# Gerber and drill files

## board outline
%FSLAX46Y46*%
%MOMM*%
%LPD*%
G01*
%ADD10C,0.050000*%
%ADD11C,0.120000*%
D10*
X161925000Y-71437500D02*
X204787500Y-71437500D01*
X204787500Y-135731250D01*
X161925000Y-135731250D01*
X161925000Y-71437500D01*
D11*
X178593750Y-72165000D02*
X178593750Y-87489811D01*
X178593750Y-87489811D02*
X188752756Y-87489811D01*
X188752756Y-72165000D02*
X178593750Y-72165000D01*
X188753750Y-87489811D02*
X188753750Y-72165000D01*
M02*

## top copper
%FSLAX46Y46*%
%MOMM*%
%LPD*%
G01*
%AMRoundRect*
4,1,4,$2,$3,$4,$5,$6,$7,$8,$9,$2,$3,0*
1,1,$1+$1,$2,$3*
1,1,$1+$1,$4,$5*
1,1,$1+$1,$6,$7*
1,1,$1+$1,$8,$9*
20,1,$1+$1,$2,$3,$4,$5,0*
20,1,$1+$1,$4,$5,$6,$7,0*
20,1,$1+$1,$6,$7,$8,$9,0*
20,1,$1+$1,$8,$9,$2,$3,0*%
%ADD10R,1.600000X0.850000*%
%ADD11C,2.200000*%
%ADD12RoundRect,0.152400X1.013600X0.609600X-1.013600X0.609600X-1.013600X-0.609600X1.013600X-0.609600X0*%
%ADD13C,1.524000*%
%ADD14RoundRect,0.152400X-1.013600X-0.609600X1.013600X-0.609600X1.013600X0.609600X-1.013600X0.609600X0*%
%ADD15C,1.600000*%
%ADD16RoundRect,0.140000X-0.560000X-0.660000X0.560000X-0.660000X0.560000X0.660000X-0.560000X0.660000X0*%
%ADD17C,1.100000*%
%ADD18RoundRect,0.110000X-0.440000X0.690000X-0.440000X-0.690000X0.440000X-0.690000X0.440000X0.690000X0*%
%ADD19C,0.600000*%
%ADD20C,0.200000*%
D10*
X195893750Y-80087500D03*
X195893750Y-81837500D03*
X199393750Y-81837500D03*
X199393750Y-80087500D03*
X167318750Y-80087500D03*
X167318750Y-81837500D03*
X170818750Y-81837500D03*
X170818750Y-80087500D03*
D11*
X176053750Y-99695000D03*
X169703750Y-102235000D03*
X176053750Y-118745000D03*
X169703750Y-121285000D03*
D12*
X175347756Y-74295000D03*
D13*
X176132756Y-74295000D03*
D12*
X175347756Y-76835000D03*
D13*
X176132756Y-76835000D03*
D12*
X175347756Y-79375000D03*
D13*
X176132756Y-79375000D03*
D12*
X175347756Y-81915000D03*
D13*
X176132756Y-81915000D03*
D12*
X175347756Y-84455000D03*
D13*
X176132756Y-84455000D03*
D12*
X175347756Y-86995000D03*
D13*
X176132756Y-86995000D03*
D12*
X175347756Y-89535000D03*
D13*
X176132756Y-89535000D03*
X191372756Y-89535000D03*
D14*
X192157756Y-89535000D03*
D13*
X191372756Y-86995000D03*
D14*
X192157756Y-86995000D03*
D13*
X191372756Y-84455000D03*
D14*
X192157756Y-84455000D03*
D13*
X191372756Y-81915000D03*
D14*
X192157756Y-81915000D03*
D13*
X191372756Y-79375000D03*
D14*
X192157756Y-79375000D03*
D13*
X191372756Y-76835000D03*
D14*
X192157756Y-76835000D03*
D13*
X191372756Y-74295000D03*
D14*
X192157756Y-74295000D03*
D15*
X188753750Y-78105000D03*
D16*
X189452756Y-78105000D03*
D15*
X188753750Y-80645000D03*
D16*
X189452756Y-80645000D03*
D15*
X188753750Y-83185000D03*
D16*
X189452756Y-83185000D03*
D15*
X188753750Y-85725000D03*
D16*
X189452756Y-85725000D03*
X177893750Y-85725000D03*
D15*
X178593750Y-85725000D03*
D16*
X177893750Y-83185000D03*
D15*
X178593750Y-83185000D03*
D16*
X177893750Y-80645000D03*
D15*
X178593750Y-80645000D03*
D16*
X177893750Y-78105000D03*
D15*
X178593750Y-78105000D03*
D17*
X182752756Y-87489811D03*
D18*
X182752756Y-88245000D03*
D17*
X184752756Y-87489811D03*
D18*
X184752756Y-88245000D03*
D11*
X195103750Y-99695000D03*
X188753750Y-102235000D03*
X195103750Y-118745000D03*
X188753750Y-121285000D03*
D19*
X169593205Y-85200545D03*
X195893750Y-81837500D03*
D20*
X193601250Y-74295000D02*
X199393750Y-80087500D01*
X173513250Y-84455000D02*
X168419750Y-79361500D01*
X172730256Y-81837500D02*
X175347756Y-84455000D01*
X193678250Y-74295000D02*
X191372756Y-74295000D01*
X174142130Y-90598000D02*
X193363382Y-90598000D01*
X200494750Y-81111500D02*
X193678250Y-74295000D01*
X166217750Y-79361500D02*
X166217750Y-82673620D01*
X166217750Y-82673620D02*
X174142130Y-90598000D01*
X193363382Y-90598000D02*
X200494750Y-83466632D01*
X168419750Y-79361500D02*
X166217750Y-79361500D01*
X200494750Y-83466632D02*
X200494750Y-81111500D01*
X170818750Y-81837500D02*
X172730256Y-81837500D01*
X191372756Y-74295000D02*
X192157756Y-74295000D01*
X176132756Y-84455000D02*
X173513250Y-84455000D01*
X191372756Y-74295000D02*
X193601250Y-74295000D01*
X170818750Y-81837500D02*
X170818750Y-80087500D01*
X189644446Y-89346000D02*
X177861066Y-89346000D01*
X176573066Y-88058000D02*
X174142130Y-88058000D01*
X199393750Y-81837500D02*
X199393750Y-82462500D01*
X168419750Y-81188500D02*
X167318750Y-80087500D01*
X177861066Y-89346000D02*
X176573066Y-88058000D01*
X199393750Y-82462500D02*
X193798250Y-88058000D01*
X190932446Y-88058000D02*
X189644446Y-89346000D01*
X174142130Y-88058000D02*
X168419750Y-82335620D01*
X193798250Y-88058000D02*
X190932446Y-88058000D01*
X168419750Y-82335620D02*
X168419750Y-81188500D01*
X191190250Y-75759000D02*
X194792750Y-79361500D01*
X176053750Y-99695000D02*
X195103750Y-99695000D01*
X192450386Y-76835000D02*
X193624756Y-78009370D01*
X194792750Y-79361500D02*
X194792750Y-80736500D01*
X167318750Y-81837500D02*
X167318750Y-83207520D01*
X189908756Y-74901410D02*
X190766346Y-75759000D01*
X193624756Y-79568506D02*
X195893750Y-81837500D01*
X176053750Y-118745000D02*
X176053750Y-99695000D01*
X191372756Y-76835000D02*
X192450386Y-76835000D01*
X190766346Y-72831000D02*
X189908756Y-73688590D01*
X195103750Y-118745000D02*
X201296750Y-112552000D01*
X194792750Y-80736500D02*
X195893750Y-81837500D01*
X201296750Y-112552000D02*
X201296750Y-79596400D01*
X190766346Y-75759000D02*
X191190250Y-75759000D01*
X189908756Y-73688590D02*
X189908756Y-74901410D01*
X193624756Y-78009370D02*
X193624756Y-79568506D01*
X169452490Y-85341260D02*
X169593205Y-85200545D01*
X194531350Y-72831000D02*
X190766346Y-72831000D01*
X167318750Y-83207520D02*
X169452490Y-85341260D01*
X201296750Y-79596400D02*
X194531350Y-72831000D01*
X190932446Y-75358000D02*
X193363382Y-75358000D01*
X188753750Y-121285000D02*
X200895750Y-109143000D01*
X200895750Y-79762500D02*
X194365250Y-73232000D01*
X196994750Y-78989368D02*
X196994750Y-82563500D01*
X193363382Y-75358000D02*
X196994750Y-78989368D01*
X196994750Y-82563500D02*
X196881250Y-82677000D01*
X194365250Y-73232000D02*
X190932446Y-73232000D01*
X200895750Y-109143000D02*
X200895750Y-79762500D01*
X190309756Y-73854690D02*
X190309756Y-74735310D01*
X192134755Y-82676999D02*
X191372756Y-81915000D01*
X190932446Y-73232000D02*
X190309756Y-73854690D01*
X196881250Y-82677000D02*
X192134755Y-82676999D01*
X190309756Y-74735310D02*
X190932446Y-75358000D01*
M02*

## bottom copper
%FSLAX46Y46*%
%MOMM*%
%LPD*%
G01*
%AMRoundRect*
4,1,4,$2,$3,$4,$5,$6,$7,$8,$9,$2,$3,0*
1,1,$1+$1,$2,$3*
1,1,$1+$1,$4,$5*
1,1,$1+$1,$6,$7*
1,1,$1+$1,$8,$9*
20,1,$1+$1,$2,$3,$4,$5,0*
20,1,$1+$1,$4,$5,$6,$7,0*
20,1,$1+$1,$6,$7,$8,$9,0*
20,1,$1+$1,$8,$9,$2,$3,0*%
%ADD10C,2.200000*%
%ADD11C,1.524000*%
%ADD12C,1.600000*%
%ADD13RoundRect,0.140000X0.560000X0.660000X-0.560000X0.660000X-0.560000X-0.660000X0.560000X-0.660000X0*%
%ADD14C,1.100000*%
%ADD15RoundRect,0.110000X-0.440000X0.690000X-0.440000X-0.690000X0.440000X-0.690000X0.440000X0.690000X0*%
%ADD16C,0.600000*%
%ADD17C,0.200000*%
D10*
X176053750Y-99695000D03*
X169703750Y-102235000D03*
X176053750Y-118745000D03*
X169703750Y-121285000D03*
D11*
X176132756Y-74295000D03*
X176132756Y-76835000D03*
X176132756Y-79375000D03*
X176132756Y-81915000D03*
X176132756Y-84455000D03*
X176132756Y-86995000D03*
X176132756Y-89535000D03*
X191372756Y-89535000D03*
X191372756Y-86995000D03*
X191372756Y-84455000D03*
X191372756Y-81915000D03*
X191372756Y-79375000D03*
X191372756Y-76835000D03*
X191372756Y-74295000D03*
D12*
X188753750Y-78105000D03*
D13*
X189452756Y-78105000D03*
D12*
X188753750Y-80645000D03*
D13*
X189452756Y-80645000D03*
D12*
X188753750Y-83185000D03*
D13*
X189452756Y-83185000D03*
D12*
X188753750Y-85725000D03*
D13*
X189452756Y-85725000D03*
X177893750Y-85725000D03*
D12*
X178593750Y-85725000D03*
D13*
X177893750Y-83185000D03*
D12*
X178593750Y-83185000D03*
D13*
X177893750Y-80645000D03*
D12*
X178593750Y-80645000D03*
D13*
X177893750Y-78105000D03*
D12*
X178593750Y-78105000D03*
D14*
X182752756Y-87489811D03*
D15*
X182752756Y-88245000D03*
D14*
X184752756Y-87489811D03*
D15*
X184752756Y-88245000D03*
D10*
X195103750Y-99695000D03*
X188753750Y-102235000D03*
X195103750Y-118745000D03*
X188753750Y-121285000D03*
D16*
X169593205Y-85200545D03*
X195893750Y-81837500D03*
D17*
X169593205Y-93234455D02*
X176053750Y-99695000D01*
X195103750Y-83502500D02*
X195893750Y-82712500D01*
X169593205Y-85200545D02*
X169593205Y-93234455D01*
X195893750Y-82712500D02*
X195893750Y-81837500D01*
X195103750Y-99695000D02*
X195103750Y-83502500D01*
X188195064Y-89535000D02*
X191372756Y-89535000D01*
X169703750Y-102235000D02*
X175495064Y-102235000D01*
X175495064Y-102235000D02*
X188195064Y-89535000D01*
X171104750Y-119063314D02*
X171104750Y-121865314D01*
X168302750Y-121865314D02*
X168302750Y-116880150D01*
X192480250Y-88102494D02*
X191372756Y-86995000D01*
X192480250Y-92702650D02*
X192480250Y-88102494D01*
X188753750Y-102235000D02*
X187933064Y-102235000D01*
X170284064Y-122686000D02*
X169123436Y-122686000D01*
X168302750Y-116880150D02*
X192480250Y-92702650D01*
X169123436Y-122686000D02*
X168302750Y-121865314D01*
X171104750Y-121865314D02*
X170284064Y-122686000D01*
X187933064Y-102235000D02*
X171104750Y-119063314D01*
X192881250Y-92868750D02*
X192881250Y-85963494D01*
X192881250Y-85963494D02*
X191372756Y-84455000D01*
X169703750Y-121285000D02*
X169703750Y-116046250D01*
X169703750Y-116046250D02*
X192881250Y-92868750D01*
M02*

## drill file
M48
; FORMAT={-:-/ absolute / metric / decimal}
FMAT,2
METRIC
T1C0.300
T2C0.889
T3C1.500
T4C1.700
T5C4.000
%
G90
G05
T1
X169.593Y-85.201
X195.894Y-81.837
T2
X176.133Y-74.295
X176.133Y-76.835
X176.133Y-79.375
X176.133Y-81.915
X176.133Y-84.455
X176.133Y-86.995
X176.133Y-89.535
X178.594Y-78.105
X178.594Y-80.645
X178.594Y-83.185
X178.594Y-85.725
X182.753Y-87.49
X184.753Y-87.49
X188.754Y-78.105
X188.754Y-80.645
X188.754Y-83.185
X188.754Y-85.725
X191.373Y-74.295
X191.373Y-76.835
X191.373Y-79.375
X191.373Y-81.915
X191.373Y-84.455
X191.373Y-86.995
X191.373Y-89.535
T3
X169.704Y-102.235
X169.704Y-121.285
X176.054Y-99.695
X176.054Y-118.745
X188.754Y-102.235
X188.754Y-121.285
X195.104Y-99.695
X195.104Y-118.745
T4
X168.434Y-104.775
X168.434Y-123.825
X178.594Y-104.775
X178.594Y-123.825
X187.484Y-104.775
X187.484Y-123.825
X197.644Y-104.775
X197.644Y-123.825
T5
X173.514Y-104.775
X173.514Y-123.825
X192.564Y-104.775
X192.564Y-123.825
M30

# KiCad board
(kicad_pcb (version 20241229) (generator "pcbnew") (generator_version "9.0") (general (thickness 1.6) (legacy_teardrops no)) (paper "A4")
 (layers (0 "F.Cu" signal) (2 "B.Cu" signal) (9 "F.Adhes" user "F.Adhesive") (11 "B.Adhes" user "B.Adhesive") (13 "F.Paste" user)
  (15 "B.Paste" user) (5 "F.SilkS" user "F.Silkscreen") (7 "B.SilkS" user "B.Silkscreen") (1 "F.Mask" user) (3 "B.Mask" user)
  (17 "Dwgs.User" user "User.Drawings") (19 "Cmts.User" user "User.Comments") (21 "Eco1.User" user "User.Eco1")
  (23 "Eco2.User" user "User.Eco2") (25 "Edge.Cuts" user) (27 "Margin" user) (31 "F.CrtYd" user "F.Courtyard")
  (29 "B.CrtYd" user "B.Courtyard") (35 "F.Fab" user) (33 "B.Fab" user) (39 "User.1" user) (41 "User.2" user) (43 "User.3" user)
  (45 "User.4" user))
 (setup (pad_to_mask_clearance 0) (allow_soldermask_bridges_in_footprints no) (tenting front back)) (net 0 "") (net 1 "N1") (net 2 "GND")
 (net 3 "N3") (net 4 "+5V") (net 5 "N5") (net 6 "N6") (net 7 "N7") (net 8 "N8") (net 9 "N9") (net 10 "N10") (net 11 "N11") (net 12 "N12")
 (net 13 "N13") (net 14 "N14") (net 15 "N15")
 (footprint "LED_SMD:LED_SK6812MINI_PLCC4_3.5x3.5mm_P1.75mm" (layer "F.Cu") (at 197.64375 80.9625)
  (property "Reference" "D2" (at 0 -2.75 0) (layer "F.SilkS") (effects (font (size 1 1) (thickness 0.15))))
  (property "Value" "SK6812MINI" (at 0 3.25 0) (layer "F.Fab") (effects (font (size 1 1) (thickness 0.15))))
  (pad "1" smd rect (at -1.75 -0.875) (size 1.6 0.85) (layers "F.Cu" "F.Mask" "F.Paste") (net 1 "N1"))
  (pad "2" smd rect (at -1.75 0.875) (size 1.6 0.85) (layers "F.Cu" "F.Mask" "F.Paste") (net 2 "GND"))
  (pad "3" smd rect (at 1.75 0.875) (size 1.6 0.85) (layers "F.Cu" "F.Mask" "F.Paste") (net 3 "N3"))
  (pad "4" smd rect (at 1.75 -0.875) (size 1.6 0.85) (layers "F.Cu" "F.Mask" "F.Paste") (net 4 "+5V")))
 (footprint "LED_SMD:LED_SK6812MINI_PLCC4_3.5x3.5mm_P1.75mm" (layer "F.Cu") (at 169.06875 80.9625)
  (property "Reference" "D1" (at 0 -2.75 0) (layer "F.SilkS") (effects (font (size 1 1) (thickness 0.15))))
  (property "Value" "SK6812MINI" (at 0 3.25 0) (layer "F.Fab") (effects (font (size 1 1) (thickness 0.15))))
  (pad "1" smd rect (at -1.75 -0.875) (size 1.6 0.85) (layers "F.Cu" "F.Mask" "F.Paste") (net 3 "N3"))
  (pad "2" smd rect (at -1.75 0.875) (size 1.6 0.85) (layers "F.Cu" "F.Mask" "F.Paste") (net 2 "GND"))
  (pad "3" smd rect (at 1.75 0.875) (size 1.6 0.85) (layers "F.Cu" "F.Mask" "F.Paste") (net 4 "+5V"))
  (pad "4" smd rect (at 1.75 -0.875) (size 1.6 0.85) (layers "F.Cu" "F.Mask" "F.Paste") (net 4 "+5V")))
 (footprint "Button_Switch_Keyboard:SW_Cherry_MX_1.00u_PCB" (layer "F.Cu") (at 176.05375 99.695)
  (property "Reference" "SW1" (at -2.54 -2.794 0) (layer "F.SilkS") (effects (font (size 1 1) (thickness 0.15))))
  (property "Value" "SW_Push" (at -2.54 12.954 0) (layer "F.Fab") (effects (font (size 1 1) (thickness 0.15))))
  (pad "" np_thru_hole circle (at -7.62 5.08) (size 1.7 1.7) (drill 1.7) (layers "*.Cu" "*.Mask"))
  (pad "" np_thru_hole circle (at -2.54 5.08) (size 4 4) (drill 4) (layers "*.Cu" "*.Mask"))
  (pad "" np_thru_hole circle (at 2.54 5.08) (size 1.7 1.7) (drill 1.7) (layers "*.Cu" "*.Mask"))
  (pad "1" thru_hole circle (at 0 0) (size 2.2 2.2) (drill 1.5) (layers "*.Cu" "*.Mask") (remove_unused_layers no) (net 2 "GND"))
  (pad "2" thru_hole circle (at -6.35 2.54) (size 2.2 2.2) (drill 1.5) (layers "*.Cu" "*.Mask") (remove_unused_layers no) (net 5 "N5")))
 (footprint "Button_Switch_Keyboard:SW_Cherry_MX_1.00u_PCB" (layer "F.Cu") (at 176.05375 118.745)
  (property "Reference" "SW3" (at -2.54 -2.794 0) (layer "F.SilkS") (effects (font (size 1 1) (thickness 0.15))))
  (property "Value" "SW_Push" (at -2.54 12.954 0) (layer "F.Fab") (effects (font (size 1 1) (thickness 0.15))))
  (pad "" np_thru_hole circle (at -7.62 5.08) (size 1.7 1.7) (drill 1.7) (layers "*.Cu" "*.Mask"))
  (pad "" np_thru_hole circle (at -2.54 5.08) (size 4 4) (drill 4) (layers "*.Cu" "*.Mask"))
  (pad "" np_thru_hole circle (at 2.54 5.08) (size 1.7 1.7) (drill 1.7) (layers "*.Cu" "*.Mask"))
  (pad "1" thru_hole circle (at 0 0) (size 2.2 2.2) (drill 1.5) (layers "*.Cu" "*.Mask") (remove_unused_layers no) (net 2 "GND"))
  (pad "2" thru_hole circle (at -6.35 2.54) (size 2.2 2.2) (drill 1.5) (layers "*.Cu" "*.Mask") (remove_unused_layers no) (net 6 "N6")))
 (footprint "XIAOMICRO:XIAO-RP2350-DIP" (layer "F.Cu") (at 183.75375 81.8515)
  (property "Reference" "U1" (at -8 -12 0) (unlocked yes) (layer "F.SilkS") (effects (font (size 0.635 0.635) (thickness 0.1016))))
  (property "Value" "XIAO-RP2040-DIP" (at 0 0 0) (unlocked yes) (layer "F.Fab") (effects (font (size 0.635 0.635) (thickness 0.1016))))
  (fp_line (start -5.16 -9.6865) (end -5.16 5.638311) (stroke (width 0.12) (type default)) (layer "Edge.Cuts"))
  (fp_line (start -5.16 5.638311) (end 4.999006 5.638311) (stroke (width 0.12) (type default)) (layer "Edge.Cuts"))
  (fp_line (start 4.999006 -9.6865) (end -5.16 -9.6865) (stroke (width 0.12) (type default)) (layer "Edge.Cuts"))
  (fp_line (start 5 5.638311) (end 5 -9.6865) (stroke (width 0.12) (type default)) (layer "Edge.Cuts"))
  (pad "1" smd roundrect (at -8.405994 -7.5565 180) (size 2.332 1.524) (layers "F.Cu" "F.Mask") (roundrect_rratio 0.1) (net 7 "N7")
   (thermal_bridge_angle 45))
  (pad "1" thru_hole circle (at -7.620994 -7.5565 180) (size 1.524 1.524) (drill 0.889) (layers "*.Cu" "*.Mask") (remove_unused_layers no)
   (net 7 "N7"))
  (pad "2" smd roundrect (at -8.405994 -5.0165 180) (size 2.332 1.524) (layers "F.Cu" "F.Mask") (roundrect_rratio 0.1) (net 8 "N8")
   (thermal_bridge_angle 45))
  (pad "2" thru_hole circle (at -7.620994 -5.0165 180) (size 1.524 1.524) (drill 0.889) (layers "*.Cu" "*.Mask") (remove_unused_layers no)
   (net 8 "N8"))
  (pad "3" smd roundrect (at -8.405994 -2.4765 180) (size 2.332 1.524) (layers "F.Cu" "F.Mask") (roundrect_rratio 0.1) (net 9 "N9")
   (thermal_bridge_angle 45))
  (pad "3" thru_hole circle (at -7.620994 -2.4765 180) (size 1.524 1.524) (drill 0.889) (layers "*.Cu" "*.Mask") (remove_unused_layers no)
   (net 9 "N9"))
  (pad "4" smd roundrect (at -8.405994 0.0635 180) (size 2.332 1.524) (layers "F.Cu" "F.Mask") (roundrect_rratio 0.1) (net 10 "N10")
   (thermal_bridge_angle 45))
  (pad "4" thru_hole circle (at -7.620994 0.0635 180) (size 1.524 1.524) (drill 0.889) (layers "*.Cu" "*.Mask") (remove_unused_layers no)
   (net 10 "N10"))
  (pad "5" smd roundrect (at -8.405994 2.6035 180) (size 2.332 1.524) (layers "F.Cu" "F.Mask") (roundrect_rratio 0.1) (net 4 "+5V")
   (thermal_bridge_angle 45))
  (pad "5" thru_hole circle (at -7.620994 2.6035 180) (size 1.524 1.524) (drill 0.889) (layers "*.Cu" "*.Mask") (remove_unused_layers no)
   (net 4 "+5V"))
  (pad "6" smd roundrect (at -8.405994 5.1435 180) (size 2.332 1.524) (layers "F.Cu" "F.Mask") (roundrect_rratio 0.1) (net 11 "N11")
   (thermal_bridge_angle 45))
  (pad "6" thru_hole circle (at -7.620994 5.1435 180) (size 1.524 1.524) (drill 0.889) (layers "*.Cu" "*.Mask") (remove_unused_layers no)
   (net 11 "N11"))
  (pad "7" smd roundrect (at -8.405994 7.6835 180) (size 2.332 1.524) (layers "F.Cu" "F.Mask") (roundrect_rratio 0.1) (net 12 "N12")
   (thermal_bridge_angle 45))
  (pad "7" thru_hole circle (at -7.620994 7.6835 180) (size 1.524 1.524) (drill 0.889) (layers "*.Cu" "*.Mask") (remove_unused_layers no)
   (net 12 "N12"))
  (pad "8" thru_hole circle (at 7.619006 7.6835) (size 1.524 1.524) (drill 0.889) (layers "*.Cu" "*.Mask") (remove_unused_layers no)
   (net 5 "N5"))
  (pad "8" smd roundrect (at 8.404006 7.6835) (size 2.332 1.524) (layers "F.Cu" "F.Mask") (roundrect_rratio 0.1) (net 5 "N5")
   (thermal_bridge_angle 45))
  (pad "9" thru_hole circle (at 7.619006 5.1435) (size 1.524 1.524) (drill 0.889) (layers "*.Cu" "*.Mask") (remove_unused_layers no)
   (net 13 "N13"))
  (pad "9" smd roundrect (at 8.404006 5.1435) (size 2.332 1.524) (layers "F.Cu" "F.Mask") (roundrect_rratio 0.1) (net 13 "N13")
   (thermal_bridge_angle 45))
  (pad "10" thru_hole circle (at 7.619006 2.6035) (size 1.524 1.524) (drill 0.889) (layers "*.Cu" "*.Mask") (remove_unused_layers no)
   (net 6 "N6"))
  (pad "10" smd roundrect (at 8.404006 2.6035) (size 2.332 1.524) (layers "F.Cu" "F.Mask") (roundrect_rratio 0.1) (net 6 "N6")
   (thermal_bridge_angle 45))
  (pad "11" thru_hole circle (at 7.619006 0.0635) (size 1.524 1.524) (drill 0.889) (layers "*.Cu" "*.Mask") (remove_unused_layers no)
   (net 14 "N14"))
  (pad "11" smd roundrect (at 8.404006 0.0635) (size 2.332 1.524) (layers "F.Cu" "F.Mask") (roundrect_rratio 0.1) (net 14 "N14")
   (thermal_bridge_angle 45))
  (pad "12" thru_hole circle (at 7.619006 -2.4765) (size 1.524 1.524) (drill 0.889) (layers "*.Cu" "*.Mask") (remove_unused_layers no)
   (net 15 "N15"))
  (pad "12" smd roundrect (at 8.404006 -2.4765) (size 2.332 1.524) (layers "F.Cu" "F.Mask") (roundrect_rratio 0.1) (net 15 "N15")
   (thermal_bridge_angle 45))
  (pad "13" thru_hole circle (at 7.619006 -5.0165) (size 1.524 1.524) (drill 0.889) (layers "*.Cu" "*.Mask") (remove_unused_layers no)
   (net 2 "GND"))
  (pad "13" smd roundrect (at 8.404006 -5.0165) (size 2.332 1.524) (layers "F.Cu" "F.Mask") (roundrect_rratio 0.1) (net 2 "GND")
   (thermal_bridge_angle 45))
  (pad "14" thru_hole circle (at 7.619006 -7.5565) (size 1.524 1.524) (drill 0.889) (layers "*.Cu" "*.Mask") (remove_unused_layers no)
   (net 4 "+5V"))
  (pad "14" smd roundrect (at 8.404006 -7.5565) (size 2.332 1.524) (layers "F.Cu" "F.Mask") (roundrect_rratio 0.1) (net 4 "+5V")
   (thermal_bridge_angle 45))
  (pad "15" thru_hole circle (at 5 -3.7465 180) (size 1.6 1.6) (drill 0.889) (layers "*.Cu" "*.Mask") (remove_unused_layers no))
  (pad "15" smd roundrect (at 5.699006 -3.7465) (size 1.4 1.6) (layers "F.Cu" "F.Mask") (roundrect_rratio 0.1) (thermal_bridge_angle 45))
  (pad "15" smd roundrect (at 5.699006 -3.7465 180) (size 1.4 1.6) (layers "B.Cu" "B.Mask" "B.Paste") (roundrect_rratio 0.1)
   (thermal_bridge_angle 45))
  (pad "16" thru_hole circle (at 5 -1.2065 180) (size 1.6 1.6) (drill 0.889) (layers "*.Cu" "*.Mask") (remove_unused_layers no))
  (pad "16" smd roundrect (at 5.699006 -1.2065) (size 1.4 1.6) (layers "F.Cu" "F.Mask") (roundrect_rratio 0.1) (thermal_bridge_angle 45))
  (pad "16" smd roundrect (at 5.699006 -1.2065 180) (size 1.4 1.6) (layers "B.Cu" "B.Mask" "B.Paste") (roundrect_rratio 0.1)
   (thermal_bridge_angle 45))
  (pad "17" thru_hole circle (at 5 1.3335 180) (size 1.6 1.6) (drill 0.889) (layers "*.Cu" "*.Mask") (remove_unused_layers no))
  (pad "17" smd roundrect (at 5.699006 1.3335) (size 1.4 1.6) (layers "F.Cu" "F.Mask") (roundrect_rratio 0.1) (thermal_bridge_angle 45))
  (pad "17" smd roundrect (at 5.699006 1.3335 180) (size 1.4 1.6) (layers "B.Cu" "B.Mask" "B.Paste") (roundrect_rratio 0.1)
   (thermal_bridge_angle 45))
  (pad "18" thru_hole circle (at 5 3.8735 180) (size 1.6 1.6) (drill 0.889) (layers "*.Cu" "*.Mask") (remove_unused_layers no))
  (pad "18" smd roundrect (at 5.699006 3.8735) (size 1.4 1.6) (layers "F.Cu" "F.Mask") (roundrect_rratio 0.1) (thermal_bridge_angle 45))
  (pad "18" smd roundrect (at 5.699006 3.8735 180) (size 1.4 1.6) (layers "B.Cu" "B.Mask" "B.Paste") (roundrect_rratio 0.1)
   (thermal_bridge_angle 45))
  (pad "19" smd roundrect (at -5.86 3.8735) (size 1.4 1.6) (layers "F.Cu" "F.Mask") (roundrect_rratio 0.1) (thermal_bridge_angle 45))
  (pad "19" smd roundrect (at -5.86 3.8735 180) (size 1.4 1.6) (layers "B.Cu" "B.Mask" "B.Paste") (roundrect_rratio 0.1)
   (thermal_bridge_angle 45))
  (pad "19" thru_hole circle (at -5.16 3.8735 180) (size 1.6 1.6) (drill 0.889) (layers "*.Cu" "*.Mask") (remove_unused_layers no))
  (pad "20" smd roundrect (at -5.86 1.3335) (size 1.4 1.6) (layers "F.Cu" "F.Mask") (roundrect_rratio 0.1) (thermal_bridge_angle 45))
  (pad "20" smd roundrect (at -5.86 1.3335 180) (size 1.4 1.6) (layers "B.Cu" "B.Mask" "B.Paste") (roundrect_rratio 0.1)
   (thermal_bridge_angle 45))
  (pad "20" thru_hole circle (at -5.16 1.3335 180) (size 1.6 1.6) (drill 0.889) (layers "*.Cu" "*.Mask") (remove_unused_layers no))
  (pad "21" smd roundrect (at -5.86 -1.2065) (size 1.4 1.6) (layers "F.Cu" "F.Mask") (roundrect_rratio 0.1) (thermal_bridge_angle 45))
  (pad "21" smd roundrect (at -5.86 -1.2065 180) (size 1.4 1.6) (layers "B.Cu" "B.Mask" "B.Paste") (roundrect_rratio 0.1)
   (thermal_bridge_angle 45))
  (pad "21" thru_hole circle (at -5.16 -1.2065 180) (size 1.6 1.6) (drill 0.889) (layers "*.Cu" "*.Mask") (remove_unused_layers no))
  (pad "22" smd roundrect (at -5.86 -3.7465) (size 1.4 1.6) (layers "F.Cu" "F.Mask") (roundrect_rratio 0.1) (thermal_bridge_angle 45))
  (pad "22" smd roundrect (at -5.86 -3.7465 180) (size 1.4 1.6) (layers "B.Cu" "B.Mask" "B.Paste") (roundrect_rratio 0.1)
   (thermal_bridge_angle 45))
  (pad "22" thru_hole circle (at -5.16 -3.7465 180) (size 1.6 1.6) (drill 0.889) (layers "*.Cu" "*.Mask") (remove_unused_layers no))
  (pad "23" thru_hole circle (at -1.000994 5.638311 180) (size 1.1 1.1) (drill 0.889) (layers "*.Cu" "*.Mask") (remove_unused_layers no))
  (pad "23" smd roundrect (at -1.000994 6.3935 270) (size 1.6 1.1) (layers "F.Cu" "F.Mask") (roundrect_rratio 0.1) (thermal_bridge_angle 45))
  (pad "23" smd roundrect (at -1.000994 6.3935 270) (size 1.6 1.1) (layers "B.Cu" "B.Mask" "B.Paste") (roundrect_rratio 0.1)
   (thermal_bridge_angle 45))
  (pad "24" thru_hole circle (at 0.999006 5.638311 180) (size 1.1 1.1) (drill 0.889) (layers "*.Cu" "*.Mask") (remove_unused_layers no))
  (pad "24" smd roundrect (at 0.999006 6.3935 270) (size 1.6 1.1) (layers "F.Cu" "F.Mask") (roundrect_rratio 0.1) (thermal_bridge_angle 45))
  (pad "24" smd roundrect (at 0.999006 6.3935 270) (size 1.6 1.1) (layers "B.Cu" "B.Mask" "B.Paste") (roundrect_rratio 0.1)
   (thermal_bridge_angle 45)))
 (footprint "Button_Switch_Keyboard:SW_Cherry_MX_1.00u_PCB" (layer "F.Cu") (at 195.10375 99.695)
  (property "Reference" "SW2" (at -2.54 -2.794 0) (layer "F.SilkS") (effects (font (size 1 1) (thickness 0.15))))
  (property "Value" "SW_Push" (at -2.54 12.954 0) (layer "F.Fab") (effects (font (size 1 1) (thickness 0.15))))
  (pad "" np_thru_hole circle (at -7.62 5.08) (size 1.7 1.7) (drill 1.7) (layers "*.Cu" "*.Mask"))
  (pad "" np_thru_hole circle (at -2.54 5.08) (size 4 4) (drill 4) (layers "*.Cu" "*.Mask"))
  (pad "" np_thru_hole circle (at 2.54 5.08) (size 1.7 1.7) (drill 1.7) (layers "*.Cu" "*.Mask"))
  (pad "1" thru_hole circle (at 0 0) (size 2.2 2.2) (drill 1.5) (layers "*.Cu" "*.Mask") (remove_unused_layers no) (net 2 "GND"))
  (pad "2" thru_hole circle (at -6.35 2.54) (size 2.2 2.2) (drill 1.5) (layers "*.Cu" "*.Mask") (remove_unused_layers no) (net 13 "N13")))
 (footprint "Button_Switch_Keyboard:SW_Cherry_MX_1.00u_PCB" (layer "F.Cu") (at 195.10375 118.745)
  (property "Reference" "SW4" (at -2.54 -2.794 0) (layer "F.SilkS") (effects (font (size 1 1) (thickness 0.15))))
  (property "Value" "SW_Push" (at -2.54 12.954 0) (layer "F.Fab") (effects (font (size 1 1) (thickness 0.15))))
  (pad "" np_thru_hole circle (at -7.62 5.08) (size 1.7 1.7) (drill 1.7) (layers "*.Cu" "*.Mask"))
  (pad "" np_thru_hole circle (at -2.54 5.08) (size 4 4) (drill 4) (layers "*.Cu" "*.Mask"))
  (pad "" np_thru_hole circle (at 2.54 5.08) (size 1.7 1.7) (drill 1.7) (layers "*.Cu" "*.Mask"))
  (pad "1" thru_hole circle (at 0 0) (size 2.2 2.2) (drill 1.5) (layers "*.Cu" "*.Mask") (remove_unused_layers no) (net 2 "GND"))
  (pad "2" thru_hole circle (at -6.35 2.54) (size 2.2 2.2) (drill 1.5) (layers "*.Cu" "*.Mask") (remove_unused_layers no) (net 14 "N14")))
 (gr_rect (start 161.925 71.4375) (end 204.7875 135.73125) (stroke (width 0.05) (type default)) (fill no) (layer "Edge.Cuts"))
 (segment (start 193.60125 74.295) (end 199.39375 80.0875) (width 0.2) (layer "F.Cu") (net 4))
 (segment (start 173.51325 84.455) (end 168.41975 79.3615) (width 0.2) (layer "F.Cu") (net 4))
 (segment (start 172.730256 81.8375) (end 175.347756 84.455) (width 0.2) (layer "F.Cu") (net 4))
 (segment (start 193.67825 74.295) (end 191.372756 74.295) (width 0.2) (layer "F.Cu") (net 4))
 (segment (start 174.14213 90.598) (end 193.363382 90.598) (width 0.2) (layer "F.Cu") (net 4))
 (segment (start 200.49475 81.1115) (end 193.67825 74.295) (width 0.2) (layer "F.Cu") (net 4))
 (segment (start 166.21775 79.3615) (end 166.21775 82.67362) (width 0.2) (layer "F.Cu") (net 4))
 (segment (start 166.21775 82.67362) (end 174.14213 90.598) (width 0.2) (layer "F.Cu") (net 4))
 (segment (start 193.363382 90.598) (end 200.49475 83.466632) (width 0.2) (layer "F.Cu") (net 4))
 (segment (start 168.41975 79.3615) (end 166.21775 79.3615) (width 0.2) (layer "F.Cu") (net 4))
 (segment (start 200.49475 83.466632) (end 200.49475 81.1115) (width 0.2) (layer "F.Cu") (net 4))
 (segment (start 170.81875 81.8375) (end 172.730256 81.8375) (width 0.2) (layer "F.Cu") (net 4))
 (segment (start 191.372756 74.295) (end 192.157756 74.295) (width 0.2) (layer "F.Cu") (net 4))
 (segment (start 176.132756 84.455) (end 173.51325 84.455) (width 0.2) (layer "F.Cu") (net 4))
 (segment (start 191.372756 74.295) (end 193.60125 74.295) (width 0.2) (layer "F.Cu") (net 4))
 (segment (start 170.81875 81.8375) (end 170.81875 80.0875) (width 0.2) (layer "F.Cu") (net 4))
 (segment (start 189.644446 89.346) (end 177.861066 89.346) (width 0.2) (layer "F.Cu") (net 3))
 (segment (start 176.573066 88.058) (end 174.14213 88.058) (width 0.2) (layer "F.Cu") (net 3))
 (segment (start 199.39375 81.8375) (end 199.39375 82.4625) (width 0.2) (layer "F.Cu") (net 3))
 (segment (start 168.41975 81.1885) (end 167.31875 80.0875) (width 0.2) (layer "F.Cu") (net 3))
 (segment (start 177.861066 89.346) (end 176.573066 88.058) (width 0.2) (layer "F.Cu") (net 3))
 (segment (start 199.39375 82.4625) (end 193.79825 88.058) (width 0.2) (layer "F.Cu") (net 3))
 (segment (start 190.932446 88.058) (end 189.644446 89.346) (width 0.2) (layer "F.Cu") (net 3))
 (segment (start 174.14213 88.058) (end 168.41975 82.33562) (width 0.2) (layer "F.Cu") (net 3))
 (segment (start 193.79825 88.058) (end 190.932446 88.058) (width 0.2) (layer "F.Cu") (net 3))
 (segment (start 168.41975 82.33562) (end 168.41975 81.1885) (width 0.2) (layer "F.Cu") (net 3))
 (segment (start 191.19025 75.759) (end 194.79275 79.3615) (width 0.2) (layer "F.Cu") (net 2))
 (segment (start 176.05375 99.695) (end 195.10375 99.695) (width 0.2) (layer "F.Cu") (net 2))
 (segment (start 192.450386 76.835) (end 193.624756 78.00937) (width 0.2) (layer "F.Cu") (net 2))
 (segment (start 194.79275 79.3615) (end 194.79275 80.7365) (width 0.2) (layer "F.Cu") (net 2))
 (segment (start 167.31875 81.8375) (end 167.31875 83.20752) (width 0.2) (layer "F.Cu") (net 2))
 (segment (start 189.908756 74.90141) (end 190.766346 75.759) (width 0.2) (layer "F.Cu") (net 2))
 (segment (start 193.624756 79.568506) (end 195.89375 81.8375) (width 0.2) (layer "F.Cu") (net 2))
 (segment (start 176.05375 118.745) (end 176.05375 99.695) (width 0.2) (layer "F.Cu") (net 2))
 (segment (start 191.372756 76.835) (end 192.450386 76.835) (width 0.2) (layer "F.Cu") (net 2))
 (segment (start 190.766346 72.831) (end 189.908756 73.68859) (width 0.2) (layer "F.Cu") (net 2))
 (segment (start 195.10375 118.745) (end 201.29675 112.552) (width 0.2) (layer "F.Cu") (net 2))
 (segment (start 194.79275 80.7365) (end 195.89375 81.8375) (width 0.2) (layer "F.Cu") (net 2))
 (segment (start 201.29675 112.552) (end 201.29675 79.5964) (width 0.2) (layer "F.Cu") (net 2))
 (segment (start 190.766346 75.759) (end 191.19025 75.759) (width 0.2) (layer "F.Cu") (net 2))
 (segment (start 189.908756 73.68859) (end 189.908756 74.90141) (width 0.2) (layer "F.Cu") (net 2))
 (segment (start 193.624756 78.00937) (end 193.624756 79.568506) (width 0.2) (layer "F.Cu") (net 2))
 (segment (start 169.45249 85.34126) (end 169.593205 85.200545) (width 0.2) (layer "F.Cu") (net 2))
 (segment (start 194.53135 72.831) (end 190.766346 72.831) (width 0.2) (layer "F.Cu") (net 2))
 (segment (start 167.31875 83.20752) (end 169.45249 85.34126) (width 0.2) (layer "F.Cu") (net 2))
 (segment (start 201.29675 79.5964) (end 194.53135 72.831) (width 0.2) (layer "F.Cu") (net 2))
 (via (at 169.593205 85.200545) (size 0.6) (drill 0.3) (layers "F.Cu" "B.Cu") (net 2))
 (via (at 195.89375 81.8375) (size 0.6) (drill 0.3) (layers "F.Cu" "B.Cu") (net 2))
 (segment (start 169.593205 93.234455) (end 176.05375 99.695) (width 0.2) (layer "B.Cu") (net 2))
 (segment (start 195.10375 83.5025) (end 195.89375 82.7125) (width 0.2) (layer "B.Cu") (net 2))
 (segment (start 169.593205 85.200545) (end 169.593205 93.234455) (width 0.2) (layer "B.Cu") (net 2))
 (segment (start 195.89375 82.7125) (end 195.89375 81.8375) (width 0.2) (layer "B.Cu") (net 2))
 (segment (start 195.10375 99.695) (end 195.10375 83.5025) (width 0.2) (layer "B.Cu") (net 2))
 (segment (start 188.195064 89.535) (end 191.372756 89.535) (width 0.2) (layer "B.Cu") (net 5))
 (segment (start 169.70375 102.235) (end 175.495064 102.235) (width 0.2) (layer "B.Cu") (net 5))
 (segment (start 175.495064 102.235) (end 188.195064 89.535) (width 0.2) (layer "B.Cu") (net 5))
 (segment (start 171.10475 119.063314) (end 171.10475 121.865314) (width 0.2) (layer "B.Cu") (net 13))
 (segment (start 168.30275 121.865314) (end 168.30275 116.88015) (width 0.2) (layer "B.Cu") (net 13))
 (segment (start 192.48025 88.102494) (end 191.372756 86.995) (width 0.2) (layer "B.Cu") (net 13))
 (segment (start 192.48025 92.70265) (end 192.48025 88.102494) (width 0.2) (layer "B.Cu") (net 13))
 (segment (start 188.75375 102.235) (end 187.933064 102.235) (width 0.2) (layer "B.Cu") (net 13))
 (segment (start 170.284064 122.686) (end 169.123436 122.686) (width 0.2) (layer "B.Cu") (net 13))
 (segment (start 168.30275 116.88015) (end 192.48025 92.70265) (width 0.2) (layer "B.Cu") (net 13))
 (segment (start 169.123436 122.686) (end 168.30275 121.865314) (width 0.2) (layer "B.Cu") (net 13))
 (segment (start 171.10475 121.865314) (end 170.284064 122.686) (width 0.2) (layer "B.Cu") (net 13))
 (segment (start 187.933064 102.235) (end 171.10475 119.063314) (width 0.2) (layer "B.Cu") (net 13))
 (segment (start 192.88125 92.86875) (end 192.88125 85.963494) (width 0.2) (layer "B.Cu") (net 6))
 (segment (start 192.88125 85.963494) (end 191.372756 84.455) (width 0.2) (layer "B.Cu") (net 6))
 (segment (start 169.70375 121.285) (end 169.70375 116.04625) (width 0.2) (layer "B.Cu") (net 6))
 (segment (start 169.70375 116.04625) (end 192.88125 92.86875) (width 0.2) (layer "B.Cu") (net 6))
 (segment (start 190.932446 75.358) (end 193.363382 75.358) (width 0.2) (layer "F.Cu") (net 14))
 (segment (start 188.75375 121.285) (end 200.89575 109.143) (width 0.2) (layer "F.Cu") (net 14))
 (segment (start 200.89575 79.7625) (end 194.36525 73.232) (width 0.2) (layer "F.Cu") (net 14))
 (segment (start 196.99475 78.989368) (end 196.99475 82.5635) (width 0.2) (layer "F.Cu") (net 14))
 (segment (start 193.363382 75.358) (end 196.99475 78.989368) (width 0.2) (layer "F.Cu") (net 14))
 (segment (start 196.99475 82.5635) (end 196.88125 82.677) (width 0.2) (layer "F.Cu") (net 14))
 (segment (start 194.36525 73.232) (end 190.932446 73.232) (width 0.2) (layer "F.Cu") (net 14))
 (segment (start 200.89575 109.143) (end 200.89575 79.7625) (width 0.2) (layer "F.Cu") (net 14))
 (segment (start 190.309756 73.85469) (end 190.309756 74.73531) (width 0.2) (layer "F.Cu") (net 14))
 (segment (start 192.134755 82.676999) (end 191.372756 81.915) (width 0.2) (layer "F.Cu") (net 14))
 (segment (start 190.932446 73.232) (end 190.309756 73.85469) (width 0.2) (layer "F.Cu") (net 14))
 (segment (start 196.88125 82.677) (end 192.134755 82.676999) (width 0.2) (layer "F.Cu") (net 14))
 (segment (start 190.309756 74.73531) (end 190.932446 75.358) (width 0.2) (layer "F.Cu") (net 14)))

